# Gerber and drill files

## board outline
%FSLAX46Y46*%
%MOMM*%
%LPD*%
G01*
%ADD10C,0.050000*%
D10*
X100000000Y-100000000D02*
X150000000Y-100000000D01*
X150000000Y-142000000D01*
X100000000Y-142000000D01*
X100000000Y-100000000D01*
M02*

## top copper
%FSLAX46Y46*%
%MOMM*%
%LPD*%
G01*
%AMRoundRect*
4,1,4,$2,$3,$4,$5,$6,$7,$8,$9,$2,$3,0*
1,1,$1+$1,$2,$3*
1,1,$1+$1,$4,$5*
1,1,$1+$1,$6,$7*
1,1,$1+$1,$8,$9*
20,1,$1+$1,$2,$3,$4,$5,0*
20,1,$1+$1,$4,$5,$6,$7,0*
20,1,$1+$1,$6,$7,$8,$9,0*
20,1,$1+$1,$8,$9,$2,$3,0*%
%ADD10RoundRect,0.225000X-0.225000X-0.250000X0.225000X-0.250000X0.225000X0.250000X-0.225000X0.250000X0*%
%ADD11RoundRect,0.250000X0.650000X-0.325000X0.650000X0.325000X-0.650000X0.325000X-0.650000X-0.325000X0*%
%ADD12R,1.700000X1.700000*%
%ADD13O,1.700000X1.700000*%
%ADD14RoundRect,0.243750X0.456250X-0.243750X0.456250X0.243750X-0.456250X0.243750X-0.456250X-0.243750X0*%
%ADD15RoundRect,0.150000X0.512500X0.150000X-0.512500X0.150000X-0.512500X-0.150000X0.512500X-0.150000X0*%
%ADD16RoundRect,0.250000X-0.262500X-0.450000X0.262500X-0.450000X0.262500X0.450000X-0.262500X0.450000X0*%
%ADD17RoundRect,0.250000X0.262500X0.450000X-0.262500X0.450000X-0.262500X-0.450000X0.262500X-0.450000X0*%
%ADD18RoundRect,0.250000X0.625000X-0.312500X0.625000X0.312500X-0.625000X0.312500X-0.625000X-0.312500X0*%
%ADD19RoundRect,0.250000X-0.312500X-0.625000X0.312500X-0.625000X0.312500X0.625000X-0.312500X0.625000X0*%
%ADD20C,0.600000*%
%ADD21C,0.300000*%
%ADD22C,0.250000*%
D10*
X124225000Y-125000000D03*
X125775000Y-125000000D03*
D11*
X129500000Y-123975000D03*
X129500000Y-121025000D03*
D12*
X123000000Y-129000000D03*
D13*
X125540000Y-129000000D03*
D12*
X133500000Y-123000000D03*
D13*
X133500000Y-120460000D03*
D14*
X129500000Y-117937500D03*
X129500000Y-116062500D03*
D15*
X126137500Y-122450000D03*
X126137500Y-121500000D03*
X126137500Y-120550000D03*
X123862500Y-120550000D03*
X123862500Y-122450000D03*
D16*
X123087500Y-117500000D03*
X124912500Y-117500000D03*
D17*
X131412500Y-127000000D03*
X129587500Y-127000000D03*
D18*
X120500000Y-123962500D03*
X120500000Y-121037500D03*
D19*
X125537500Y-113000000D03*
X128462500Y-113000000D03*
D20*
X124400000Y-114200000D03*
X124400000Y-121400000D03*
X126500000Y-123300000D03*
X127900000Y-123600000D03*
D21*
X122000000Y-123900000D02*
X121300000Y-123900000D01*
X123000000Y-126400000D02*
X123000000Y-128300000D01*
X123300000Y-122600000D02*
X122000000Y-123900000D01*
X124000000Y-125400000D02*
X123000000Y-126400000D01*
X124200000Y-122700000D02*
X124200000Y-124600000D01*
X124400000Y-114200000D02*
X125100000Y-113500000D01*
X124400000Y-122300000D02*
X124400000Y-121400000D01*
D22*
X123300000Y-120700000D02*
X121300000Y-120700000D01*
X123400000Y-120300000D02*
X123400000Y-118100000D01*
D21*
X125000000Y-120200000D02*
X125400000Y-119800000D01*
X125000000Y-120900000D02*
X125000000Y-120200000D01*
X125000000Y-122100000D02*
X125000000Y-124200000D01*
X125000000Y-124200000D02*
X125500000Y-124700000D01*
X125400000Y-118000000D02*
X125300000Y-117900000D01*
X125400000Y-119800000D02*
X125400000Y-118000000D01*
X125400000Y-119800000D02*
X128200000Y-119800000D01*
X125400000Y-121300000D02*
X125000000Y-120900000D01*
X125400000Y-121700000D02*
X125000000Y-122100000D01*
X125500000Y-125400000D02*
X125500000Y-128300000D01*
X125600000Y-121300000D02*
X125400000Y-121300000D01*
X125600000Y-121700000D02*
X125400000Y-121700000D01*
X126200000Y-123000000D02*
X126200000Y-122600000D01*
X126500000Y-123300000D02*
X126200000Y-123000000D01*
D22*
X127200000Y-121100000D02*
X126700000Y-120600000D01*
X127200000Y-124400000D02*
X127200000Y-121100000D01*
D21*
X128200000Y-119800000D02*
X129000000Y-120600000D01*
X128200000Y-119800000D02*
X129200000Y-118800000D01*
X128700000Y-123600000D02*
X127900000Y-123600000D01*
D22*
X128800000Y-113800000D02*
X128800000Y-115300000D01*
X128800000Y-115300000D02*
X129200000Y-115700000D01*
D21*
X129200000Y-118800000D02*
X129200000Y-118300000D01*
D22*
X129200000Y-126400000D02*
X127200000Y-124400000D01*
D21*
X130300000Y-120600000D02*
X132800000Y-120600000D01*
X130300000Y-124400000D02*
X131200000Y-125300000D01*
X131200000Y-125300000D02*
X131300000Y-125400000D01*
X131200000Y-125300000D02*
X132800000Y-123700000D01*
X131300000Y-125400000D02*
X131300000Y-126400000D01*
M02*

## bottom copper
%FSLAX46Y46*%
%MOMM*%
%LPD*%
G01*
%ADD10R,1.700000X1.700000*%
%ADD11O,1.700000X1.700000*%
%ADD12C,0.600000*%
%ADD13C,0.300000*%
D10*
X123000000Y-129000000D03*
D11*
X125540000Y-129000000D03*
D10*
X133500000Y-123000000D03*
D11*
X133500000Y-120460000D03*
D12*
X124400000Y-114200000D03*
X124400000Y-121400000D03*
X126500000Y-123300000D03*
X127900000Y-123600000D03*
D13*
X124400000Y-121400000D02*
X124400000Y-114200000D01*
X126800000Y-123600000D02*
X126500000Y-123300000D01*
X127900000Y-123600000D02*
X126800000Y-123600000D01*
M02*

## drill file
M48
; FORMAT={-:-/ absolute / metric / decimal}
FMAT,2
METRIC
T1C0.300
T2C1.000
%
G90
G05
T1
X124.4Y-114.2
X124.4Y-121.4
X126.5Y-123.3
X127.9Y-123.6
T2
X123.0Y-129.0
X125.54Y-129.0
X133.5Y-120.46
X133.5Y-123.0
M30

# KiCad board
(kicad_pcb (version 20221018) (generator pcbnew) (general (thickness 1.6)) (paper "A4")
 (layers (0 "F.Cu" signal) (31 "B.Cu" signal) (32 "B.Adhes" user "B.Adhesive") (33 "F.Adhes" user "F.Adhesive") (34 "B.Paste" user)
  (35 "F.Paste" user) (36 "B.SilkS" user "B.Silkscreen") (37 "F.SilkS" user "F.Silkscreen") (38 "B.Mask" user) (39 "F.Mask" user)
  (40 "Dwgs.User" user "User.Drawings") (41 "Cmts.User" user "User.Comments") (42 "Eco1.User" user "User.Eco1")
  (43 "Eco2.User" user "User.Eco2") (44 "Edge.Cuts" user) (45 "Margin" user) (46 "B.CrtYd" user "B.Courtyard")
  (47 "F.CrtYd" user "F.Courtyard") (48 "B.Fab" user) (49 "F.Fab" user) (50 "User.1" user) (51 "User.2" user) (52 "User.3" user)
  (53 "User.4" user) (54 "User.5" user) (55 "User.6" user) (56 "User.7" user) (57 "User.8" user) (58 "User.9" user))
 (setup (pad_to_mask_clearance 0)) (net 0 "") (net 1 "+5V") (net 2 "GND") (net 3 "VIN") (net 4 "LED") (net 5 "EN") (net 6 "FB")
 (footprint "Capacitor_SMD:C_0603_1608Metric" (layer "F.Cu") (at 125 125)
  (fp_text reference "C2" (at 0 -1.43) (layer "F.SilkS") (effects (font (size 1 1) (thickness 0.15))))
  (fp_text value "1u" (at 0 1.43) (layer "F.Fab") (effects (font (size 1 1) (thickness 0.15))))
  (pad "1" smd roundrect (at -0.775 0) (size 0.9 0.95) (layers "F.Cu" "F.Paste" "F.Mask") (roundrect_rratio 0.25) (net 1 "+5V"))
  (pad "2" smd roundrect (at 0.775 0) (size 0.9 0.95) (layers "F.Cu" "F.Paste" "F.Mask") (roundrect_rratio 0.25) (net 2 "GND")))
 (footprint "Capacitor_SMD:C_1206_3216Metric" (layer "F.Cu") (at 129.5 122.5 90)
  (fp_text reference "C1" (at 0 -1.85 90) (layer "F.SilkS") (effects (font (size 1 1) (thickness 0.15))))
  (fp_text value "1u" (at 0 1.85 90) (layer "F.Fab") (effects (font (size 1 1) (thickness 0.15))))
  (pad "1" smd roundrect (at -1.475 0 90) (size 1.15 1.8) (layers "F.Cu" "F.Paste" "F.Mask") (roundrect_rratio 0.217391) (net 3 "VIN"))
  (pad "2" smd roundrect (at 1.475 0 90) (size 1.15 1.8) (layers "F.Cu" "F.Paste" "F.Mask") (roundrect_rratio 0.217391) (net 2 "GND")))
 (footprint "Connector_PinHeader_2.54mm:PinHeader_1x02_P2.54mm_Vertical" (layer "F.Cu") (at 123 129 90)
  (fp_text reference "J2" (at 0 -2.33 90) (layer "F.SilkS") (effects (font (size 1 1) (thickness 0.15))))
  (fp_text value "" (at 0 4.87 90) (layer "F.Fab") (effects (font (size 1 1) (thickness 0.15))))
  (pad "1" thru_hole rect (at 0 0 90) (size 1.7 1.7) (drill 1) (layers "*.Cu" "*.Mask") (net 1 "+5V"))
  (pad "2" thru_hole oval (at 0 2.54 90) (size 1.7 1.7) (drill 1) (layers "*.Cu" "*.Mask") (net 2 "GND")))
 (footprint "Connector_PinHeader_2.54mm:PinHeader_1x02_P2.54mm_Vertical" (layer "F.Cu") (at 133.5 123 180)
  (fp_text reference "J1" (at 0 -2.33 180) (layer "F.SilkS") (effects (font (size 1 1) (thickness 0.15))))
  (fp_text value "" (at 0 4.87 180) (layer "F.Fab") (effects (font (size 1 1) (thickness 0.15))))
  (pad "1" thru_hole rect (at 0 0 180) (size 1.7 1.7) (drill 1) (layers "*.Cu" "*.Mask") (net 3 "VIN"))
  (pad "2" thru_hole oval (at 0 2.54 180) (size 1.7 1.7) (drill 1) (layers "*.Cu" "*.Mask") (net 2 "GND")))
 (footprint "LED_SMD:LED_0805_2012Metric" (layer "F.Cu") (at 129.5 117 90)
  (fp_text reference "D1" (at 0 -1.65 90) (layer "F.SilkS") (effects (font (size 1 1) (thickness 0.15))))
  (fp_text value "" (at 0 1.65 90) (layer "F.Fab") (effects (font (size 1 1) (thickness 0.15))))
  (pad "1" smd roundrect (at -0.9375 0 90) (size 0.975 1.4) (layers "F.Cu" "F.Paste" "F.Mask") (roundrect_rratio 0.25) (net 2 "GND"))
  (pad "2" smd roundrect (at 0.9375 0 90) (size 0.975 1.4) (layers "F.Cu" "F.Paste" "F.Mask") (roundrect_rratio 0.25) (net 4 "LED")))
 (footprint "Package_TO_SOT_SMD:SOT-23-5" (layer "F.Cu") (at 125 121.5 180)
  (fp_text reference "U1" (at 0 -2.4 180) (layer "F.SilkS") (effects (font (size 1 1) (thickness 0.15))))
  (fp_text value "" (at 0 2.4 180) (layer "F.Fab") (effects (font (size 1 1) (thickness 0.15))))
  (pad "1" smd roundrect (at -1.1375 -0.95 180) (size 1.325 0.6) (layers "F.Cu" "F.Paste" "F.Mask") (roundrect_rratio 0.25) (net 3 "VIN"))
  (pad "2" smd roundrect (at -1.1375 0 180) (size 1.325 0.6) (layers "F.Cu" "F.Paste" "F.Mask") (roundrect_rratio 0.25) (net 2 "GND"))
  (pad "3" smd roundrect (at -1.1375 0.95 180) (size 1.325 0.6) (layers "F.Cu" "F.Paste" "F.Mask") (roundrect_rratio 0.25) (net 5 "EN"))
  (pad "4" smd roundrect (at 1.1375 0.95 180) (size 1.325 0.6) (layers "F.Cu" "F.Paste" "F.Mask") (roundrect_rratio 0.25) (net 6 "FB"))
  (pad "5" smd roundrect (at 1.1375 -0.95 180) (size 1.325 0.6) (layers "F.Cu" "F.Paste" "F.Mask") (roundrect_rratio 0.25) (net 1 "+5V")))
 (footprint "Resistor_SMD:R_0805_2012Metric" (layer "F.Cu") (at 124 117.5)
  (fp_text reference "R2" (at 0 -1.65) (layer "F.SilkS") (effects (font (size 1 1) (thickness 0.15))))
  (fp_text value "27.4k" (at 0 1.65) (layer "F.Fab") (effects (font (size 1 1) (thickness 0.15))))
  (pad "1" smd roundrect (at -0.9125 0) (size 1.025 1.4) (layers "F.Cu" "F.Paste" "F.Mask") (roundrect_rratio 0.243902) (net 6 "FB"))
  (pad "2" smd roundrect (at 0.9125 0) (size 1.025 1.4) (layers "F.Cu" "F.Paste" "F.Mask") (roundrect_rratio 0.243902) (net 2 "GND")))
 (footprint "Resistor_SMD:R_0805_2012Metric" (layer "F.Cu") (at 130.5 127 180)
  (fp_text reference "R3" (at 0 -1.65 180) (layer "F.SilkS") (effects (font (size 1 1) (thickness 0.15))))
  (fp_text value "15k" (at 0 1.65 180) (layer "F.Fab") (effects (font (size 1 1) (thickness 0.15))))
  (pad "1" smd roundrect (at -0.9125 0 180) (size 1.025 1.4) (layers "F.Cu" "F.Paste" "F.Mask") (roundrect_rratio 0.243902) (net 3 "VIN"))
  (pad "2" smd roundrect (at 0.9125 0 180) (size 1.025 1.4) (layers "F.Cu" "F.Paste" "F.Mask") (roundrect_rratio 0.243902) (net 5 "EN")))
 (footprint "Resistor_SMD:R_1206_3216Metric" (layer "F.Cu") (at 120.5 122.5 90)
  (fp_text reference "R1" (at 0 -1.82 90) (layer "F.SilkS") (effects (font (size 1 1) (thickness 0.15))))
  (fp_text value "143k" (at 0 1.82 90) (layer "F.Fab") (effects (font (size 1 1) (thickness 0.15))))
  (pad "1" smd roundrect (at -1.4625 0 90) (size 1.125 1.75) (layers "F.Cu" "F.Paste" "F.Mask") (roundrect_rratio 0.222222) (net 1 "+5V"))
  (pad "2" smd roundrect (at 1.4625 0 90) (size 1.125 1.75) (layers "F.Cu" "F.Paste" "F.Mask") (roundrect_rratio 0.222222) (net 6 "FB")))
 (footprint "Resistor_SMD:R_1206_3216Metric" (layer "F.Cu") (at 127 113)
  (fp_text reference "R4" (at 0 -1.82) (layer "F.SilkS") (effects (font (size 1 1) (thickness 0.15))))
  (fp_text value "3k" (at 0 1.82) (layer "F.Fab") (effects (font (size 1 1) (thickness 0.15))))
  (pad "1" smd roundrect (at -1.4625 0) (size 1.125 1.75) (layers "F.Cu" "F.Paste" "F.Mask") (roundrect_rratio 0.222222) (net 1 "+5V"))
  (pad "2" smd roundrect (at 1.4625 0) (size 1.125 1.75) (layers "F.Cu" "F.Paste" "F.Mask") (roundrect_rratio 0.222222) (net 4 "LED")))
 (gr_rect (start 100 100) (end 150 142) (stroke (width 0.05) (type default)) (fill none) (layer "Edge.Cuts"))
 (segment (start 122 123.9) (end 121.3 123.9) (width 0.3) (layer "F.Cu") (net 1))
 (segment (start 123 126.4) (end 123 128.3) (width 0.3) (layer "F.Cu") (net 1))
 (segment (start 123.3 122.6) (end 122 123.9) (width 0.3) (layer "F.Cu") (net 1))
 (segment (start 124 125.4) (end 123 126.4) (width 0.3) (layer "F.Cu") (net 1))
 (segment (start 124.2 122.7) (end 124.2 124.6) (width 0.3) (layer "F.Cu") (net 1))
 (segment (start 124.4 114.2) (end 125.1 113.5) (width 0.3) (layer "F.Cu") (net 1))
 (segment (start 124.4 122.3) (end 124.4 121.4) (width 0.3) (layer "F.Cu") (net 1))
 (via (at 124.4 114.2) (size 0.6) (drill 0.3) (layers "F.Cu" "B.Cu") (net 1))
 (via (at 124.4 121.4) (size 0.6) (drill 0.3) (layers "F.Cu" "B.Cu") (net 1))
 (segment (start 123.3 120.7) (end 121.3 120.7) (width 0.25) (layer "F.Cu") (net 6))
 (segment (start 123.4 120.3) (end 123.4 118.1) (width 0.25) (layer "F.Cu") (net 6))
 (segment (start 124.4 121.4) (end 124.4 114.2) (width 0.3) (layer "B.Cu") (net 1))
 (segment (start 125 120.2) (end 125.4 119.8) (width 0.3) (layer "F.Cu") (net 2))
 (segment (start 125 120.9) (end 125 120.2) (width 0.3) (layer "F.Cu") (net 2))
 (segment (start 125 122.1) (end 125 124.2) (width 0.3) (layer "F.Cu") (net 2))
 (segment (start 125 124.2) (end 125.5 124.7) (width 0.3) (layer "F.Cu") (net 2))
 (segment (start 125.4 118) (end 125.3 117.9) (width 0.3) (layer "F.Cu") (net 2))
 (segment (start 125.4 119.8) (end 125.4 118) (width 0.3) (layer "F.Cu") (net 2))
 (segment (start 125.4 119.8) (end 128.2 119.8) (width 0.3) (layer "F.Cu") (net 2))
 (segment (start 125.4 121.3) (end 125 120.9) (width 0.3) (layer "F.Cu") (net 2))
 (segment (start 125.4 121.7) (end 125 122.1) (width 0.3) (layer "F.Cu") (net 2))
 (segment (start 125.5 125.4) (end 125.5 128.3) (width 0.3) (layer "F.Cu") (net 2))
 (segment (start 125.6 121.3) (end 125.4 121.3) (width 0.3) (layer "F.Cu") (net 2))
 (segment (start 125.6 121.7) (end 125.4 121.7) (width 0.3) (layer "F.Cu") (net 2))
 (segment (start 126.2 123) (end 126.2 122.6) (width 0.3) (layer "F.Cu") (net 3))
 (segment (start 126.5 123.3) (end 126.2 123) (width 0.3) (layer "F.Cu") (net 3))
 (segment (start 127.2 121.1) (end 126.7 120.6) (width 0.25) (layer "F.Cu") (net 5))
 (segment (start 127.2 124.4) (end 127.2 121.1) (width 0.25) (layer "F.Cu") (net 5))
 (segment (start 128.2 119.8) (end 129 120.6) (width 0.3) (layer "F.Cu") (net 2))
 (segment (start 128.2 119.8) (end 129.2 118.8) (width 0.3) (layer "F.Cu") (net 2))
 (segment (start 128.7 123.6) (end 127.9 123.6) (width 0.3) (layer "F.Cu") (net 3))
 (segment (start 128.8 113.8) (end 128.8 115.3) (width 0.25) (layer "F.Cu") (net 4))
 (segment (start 128.8 115.3) (end 129.2 115.7) (width 0.25) (layer "F.Cu") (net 4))
 (segment (start 129.2 118.8) (end 129.2 118.3) (width 0.3) (layer "F.Cu") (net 2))
 (segment (start 129.2 126.4) (end 127.2 124.4) (width 0.25) (layer "F.Cu") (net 5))
 (segment (start 130.3 120.6) (end 132.8 120.6) (width 0.3) (layer "F.Cu") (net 2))
 (segment (start 130.3 124.4) (end 131.2 125.3) (width 0.3) (layer "F.Cu") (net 3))
 (segment (start 131.2 125.3) (end 131.3 125.4) (width 0.3) (layer "F.Cu") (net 3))
 (segment (start 131.2 125.3) (end 132.8 123.7) (width 0.3) (layer "F.Cu") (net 3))
 (segment (start 131.3 125.4) (end 131.3 126.4) (width 0.3) (layer "F.Cu") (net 3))
 (via (at 126.5 123.3) (size 0.6) (drill 0.3) (layers "F.Cu" "B.Cu") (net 3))
 (via (at 127.9 123.6) (size 0.6) (drill 0.3) (layers "F.Cu" "B.Cu") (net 3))
 (segment (start 126.8 123.6) (end 126.5 123.3) (width 0.3) (layer "B.Cu") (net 3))
 (segment (start 127.9 123.6) (end 126.8 123.6) (width 0.3) (layer "B.Cu") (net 3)))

